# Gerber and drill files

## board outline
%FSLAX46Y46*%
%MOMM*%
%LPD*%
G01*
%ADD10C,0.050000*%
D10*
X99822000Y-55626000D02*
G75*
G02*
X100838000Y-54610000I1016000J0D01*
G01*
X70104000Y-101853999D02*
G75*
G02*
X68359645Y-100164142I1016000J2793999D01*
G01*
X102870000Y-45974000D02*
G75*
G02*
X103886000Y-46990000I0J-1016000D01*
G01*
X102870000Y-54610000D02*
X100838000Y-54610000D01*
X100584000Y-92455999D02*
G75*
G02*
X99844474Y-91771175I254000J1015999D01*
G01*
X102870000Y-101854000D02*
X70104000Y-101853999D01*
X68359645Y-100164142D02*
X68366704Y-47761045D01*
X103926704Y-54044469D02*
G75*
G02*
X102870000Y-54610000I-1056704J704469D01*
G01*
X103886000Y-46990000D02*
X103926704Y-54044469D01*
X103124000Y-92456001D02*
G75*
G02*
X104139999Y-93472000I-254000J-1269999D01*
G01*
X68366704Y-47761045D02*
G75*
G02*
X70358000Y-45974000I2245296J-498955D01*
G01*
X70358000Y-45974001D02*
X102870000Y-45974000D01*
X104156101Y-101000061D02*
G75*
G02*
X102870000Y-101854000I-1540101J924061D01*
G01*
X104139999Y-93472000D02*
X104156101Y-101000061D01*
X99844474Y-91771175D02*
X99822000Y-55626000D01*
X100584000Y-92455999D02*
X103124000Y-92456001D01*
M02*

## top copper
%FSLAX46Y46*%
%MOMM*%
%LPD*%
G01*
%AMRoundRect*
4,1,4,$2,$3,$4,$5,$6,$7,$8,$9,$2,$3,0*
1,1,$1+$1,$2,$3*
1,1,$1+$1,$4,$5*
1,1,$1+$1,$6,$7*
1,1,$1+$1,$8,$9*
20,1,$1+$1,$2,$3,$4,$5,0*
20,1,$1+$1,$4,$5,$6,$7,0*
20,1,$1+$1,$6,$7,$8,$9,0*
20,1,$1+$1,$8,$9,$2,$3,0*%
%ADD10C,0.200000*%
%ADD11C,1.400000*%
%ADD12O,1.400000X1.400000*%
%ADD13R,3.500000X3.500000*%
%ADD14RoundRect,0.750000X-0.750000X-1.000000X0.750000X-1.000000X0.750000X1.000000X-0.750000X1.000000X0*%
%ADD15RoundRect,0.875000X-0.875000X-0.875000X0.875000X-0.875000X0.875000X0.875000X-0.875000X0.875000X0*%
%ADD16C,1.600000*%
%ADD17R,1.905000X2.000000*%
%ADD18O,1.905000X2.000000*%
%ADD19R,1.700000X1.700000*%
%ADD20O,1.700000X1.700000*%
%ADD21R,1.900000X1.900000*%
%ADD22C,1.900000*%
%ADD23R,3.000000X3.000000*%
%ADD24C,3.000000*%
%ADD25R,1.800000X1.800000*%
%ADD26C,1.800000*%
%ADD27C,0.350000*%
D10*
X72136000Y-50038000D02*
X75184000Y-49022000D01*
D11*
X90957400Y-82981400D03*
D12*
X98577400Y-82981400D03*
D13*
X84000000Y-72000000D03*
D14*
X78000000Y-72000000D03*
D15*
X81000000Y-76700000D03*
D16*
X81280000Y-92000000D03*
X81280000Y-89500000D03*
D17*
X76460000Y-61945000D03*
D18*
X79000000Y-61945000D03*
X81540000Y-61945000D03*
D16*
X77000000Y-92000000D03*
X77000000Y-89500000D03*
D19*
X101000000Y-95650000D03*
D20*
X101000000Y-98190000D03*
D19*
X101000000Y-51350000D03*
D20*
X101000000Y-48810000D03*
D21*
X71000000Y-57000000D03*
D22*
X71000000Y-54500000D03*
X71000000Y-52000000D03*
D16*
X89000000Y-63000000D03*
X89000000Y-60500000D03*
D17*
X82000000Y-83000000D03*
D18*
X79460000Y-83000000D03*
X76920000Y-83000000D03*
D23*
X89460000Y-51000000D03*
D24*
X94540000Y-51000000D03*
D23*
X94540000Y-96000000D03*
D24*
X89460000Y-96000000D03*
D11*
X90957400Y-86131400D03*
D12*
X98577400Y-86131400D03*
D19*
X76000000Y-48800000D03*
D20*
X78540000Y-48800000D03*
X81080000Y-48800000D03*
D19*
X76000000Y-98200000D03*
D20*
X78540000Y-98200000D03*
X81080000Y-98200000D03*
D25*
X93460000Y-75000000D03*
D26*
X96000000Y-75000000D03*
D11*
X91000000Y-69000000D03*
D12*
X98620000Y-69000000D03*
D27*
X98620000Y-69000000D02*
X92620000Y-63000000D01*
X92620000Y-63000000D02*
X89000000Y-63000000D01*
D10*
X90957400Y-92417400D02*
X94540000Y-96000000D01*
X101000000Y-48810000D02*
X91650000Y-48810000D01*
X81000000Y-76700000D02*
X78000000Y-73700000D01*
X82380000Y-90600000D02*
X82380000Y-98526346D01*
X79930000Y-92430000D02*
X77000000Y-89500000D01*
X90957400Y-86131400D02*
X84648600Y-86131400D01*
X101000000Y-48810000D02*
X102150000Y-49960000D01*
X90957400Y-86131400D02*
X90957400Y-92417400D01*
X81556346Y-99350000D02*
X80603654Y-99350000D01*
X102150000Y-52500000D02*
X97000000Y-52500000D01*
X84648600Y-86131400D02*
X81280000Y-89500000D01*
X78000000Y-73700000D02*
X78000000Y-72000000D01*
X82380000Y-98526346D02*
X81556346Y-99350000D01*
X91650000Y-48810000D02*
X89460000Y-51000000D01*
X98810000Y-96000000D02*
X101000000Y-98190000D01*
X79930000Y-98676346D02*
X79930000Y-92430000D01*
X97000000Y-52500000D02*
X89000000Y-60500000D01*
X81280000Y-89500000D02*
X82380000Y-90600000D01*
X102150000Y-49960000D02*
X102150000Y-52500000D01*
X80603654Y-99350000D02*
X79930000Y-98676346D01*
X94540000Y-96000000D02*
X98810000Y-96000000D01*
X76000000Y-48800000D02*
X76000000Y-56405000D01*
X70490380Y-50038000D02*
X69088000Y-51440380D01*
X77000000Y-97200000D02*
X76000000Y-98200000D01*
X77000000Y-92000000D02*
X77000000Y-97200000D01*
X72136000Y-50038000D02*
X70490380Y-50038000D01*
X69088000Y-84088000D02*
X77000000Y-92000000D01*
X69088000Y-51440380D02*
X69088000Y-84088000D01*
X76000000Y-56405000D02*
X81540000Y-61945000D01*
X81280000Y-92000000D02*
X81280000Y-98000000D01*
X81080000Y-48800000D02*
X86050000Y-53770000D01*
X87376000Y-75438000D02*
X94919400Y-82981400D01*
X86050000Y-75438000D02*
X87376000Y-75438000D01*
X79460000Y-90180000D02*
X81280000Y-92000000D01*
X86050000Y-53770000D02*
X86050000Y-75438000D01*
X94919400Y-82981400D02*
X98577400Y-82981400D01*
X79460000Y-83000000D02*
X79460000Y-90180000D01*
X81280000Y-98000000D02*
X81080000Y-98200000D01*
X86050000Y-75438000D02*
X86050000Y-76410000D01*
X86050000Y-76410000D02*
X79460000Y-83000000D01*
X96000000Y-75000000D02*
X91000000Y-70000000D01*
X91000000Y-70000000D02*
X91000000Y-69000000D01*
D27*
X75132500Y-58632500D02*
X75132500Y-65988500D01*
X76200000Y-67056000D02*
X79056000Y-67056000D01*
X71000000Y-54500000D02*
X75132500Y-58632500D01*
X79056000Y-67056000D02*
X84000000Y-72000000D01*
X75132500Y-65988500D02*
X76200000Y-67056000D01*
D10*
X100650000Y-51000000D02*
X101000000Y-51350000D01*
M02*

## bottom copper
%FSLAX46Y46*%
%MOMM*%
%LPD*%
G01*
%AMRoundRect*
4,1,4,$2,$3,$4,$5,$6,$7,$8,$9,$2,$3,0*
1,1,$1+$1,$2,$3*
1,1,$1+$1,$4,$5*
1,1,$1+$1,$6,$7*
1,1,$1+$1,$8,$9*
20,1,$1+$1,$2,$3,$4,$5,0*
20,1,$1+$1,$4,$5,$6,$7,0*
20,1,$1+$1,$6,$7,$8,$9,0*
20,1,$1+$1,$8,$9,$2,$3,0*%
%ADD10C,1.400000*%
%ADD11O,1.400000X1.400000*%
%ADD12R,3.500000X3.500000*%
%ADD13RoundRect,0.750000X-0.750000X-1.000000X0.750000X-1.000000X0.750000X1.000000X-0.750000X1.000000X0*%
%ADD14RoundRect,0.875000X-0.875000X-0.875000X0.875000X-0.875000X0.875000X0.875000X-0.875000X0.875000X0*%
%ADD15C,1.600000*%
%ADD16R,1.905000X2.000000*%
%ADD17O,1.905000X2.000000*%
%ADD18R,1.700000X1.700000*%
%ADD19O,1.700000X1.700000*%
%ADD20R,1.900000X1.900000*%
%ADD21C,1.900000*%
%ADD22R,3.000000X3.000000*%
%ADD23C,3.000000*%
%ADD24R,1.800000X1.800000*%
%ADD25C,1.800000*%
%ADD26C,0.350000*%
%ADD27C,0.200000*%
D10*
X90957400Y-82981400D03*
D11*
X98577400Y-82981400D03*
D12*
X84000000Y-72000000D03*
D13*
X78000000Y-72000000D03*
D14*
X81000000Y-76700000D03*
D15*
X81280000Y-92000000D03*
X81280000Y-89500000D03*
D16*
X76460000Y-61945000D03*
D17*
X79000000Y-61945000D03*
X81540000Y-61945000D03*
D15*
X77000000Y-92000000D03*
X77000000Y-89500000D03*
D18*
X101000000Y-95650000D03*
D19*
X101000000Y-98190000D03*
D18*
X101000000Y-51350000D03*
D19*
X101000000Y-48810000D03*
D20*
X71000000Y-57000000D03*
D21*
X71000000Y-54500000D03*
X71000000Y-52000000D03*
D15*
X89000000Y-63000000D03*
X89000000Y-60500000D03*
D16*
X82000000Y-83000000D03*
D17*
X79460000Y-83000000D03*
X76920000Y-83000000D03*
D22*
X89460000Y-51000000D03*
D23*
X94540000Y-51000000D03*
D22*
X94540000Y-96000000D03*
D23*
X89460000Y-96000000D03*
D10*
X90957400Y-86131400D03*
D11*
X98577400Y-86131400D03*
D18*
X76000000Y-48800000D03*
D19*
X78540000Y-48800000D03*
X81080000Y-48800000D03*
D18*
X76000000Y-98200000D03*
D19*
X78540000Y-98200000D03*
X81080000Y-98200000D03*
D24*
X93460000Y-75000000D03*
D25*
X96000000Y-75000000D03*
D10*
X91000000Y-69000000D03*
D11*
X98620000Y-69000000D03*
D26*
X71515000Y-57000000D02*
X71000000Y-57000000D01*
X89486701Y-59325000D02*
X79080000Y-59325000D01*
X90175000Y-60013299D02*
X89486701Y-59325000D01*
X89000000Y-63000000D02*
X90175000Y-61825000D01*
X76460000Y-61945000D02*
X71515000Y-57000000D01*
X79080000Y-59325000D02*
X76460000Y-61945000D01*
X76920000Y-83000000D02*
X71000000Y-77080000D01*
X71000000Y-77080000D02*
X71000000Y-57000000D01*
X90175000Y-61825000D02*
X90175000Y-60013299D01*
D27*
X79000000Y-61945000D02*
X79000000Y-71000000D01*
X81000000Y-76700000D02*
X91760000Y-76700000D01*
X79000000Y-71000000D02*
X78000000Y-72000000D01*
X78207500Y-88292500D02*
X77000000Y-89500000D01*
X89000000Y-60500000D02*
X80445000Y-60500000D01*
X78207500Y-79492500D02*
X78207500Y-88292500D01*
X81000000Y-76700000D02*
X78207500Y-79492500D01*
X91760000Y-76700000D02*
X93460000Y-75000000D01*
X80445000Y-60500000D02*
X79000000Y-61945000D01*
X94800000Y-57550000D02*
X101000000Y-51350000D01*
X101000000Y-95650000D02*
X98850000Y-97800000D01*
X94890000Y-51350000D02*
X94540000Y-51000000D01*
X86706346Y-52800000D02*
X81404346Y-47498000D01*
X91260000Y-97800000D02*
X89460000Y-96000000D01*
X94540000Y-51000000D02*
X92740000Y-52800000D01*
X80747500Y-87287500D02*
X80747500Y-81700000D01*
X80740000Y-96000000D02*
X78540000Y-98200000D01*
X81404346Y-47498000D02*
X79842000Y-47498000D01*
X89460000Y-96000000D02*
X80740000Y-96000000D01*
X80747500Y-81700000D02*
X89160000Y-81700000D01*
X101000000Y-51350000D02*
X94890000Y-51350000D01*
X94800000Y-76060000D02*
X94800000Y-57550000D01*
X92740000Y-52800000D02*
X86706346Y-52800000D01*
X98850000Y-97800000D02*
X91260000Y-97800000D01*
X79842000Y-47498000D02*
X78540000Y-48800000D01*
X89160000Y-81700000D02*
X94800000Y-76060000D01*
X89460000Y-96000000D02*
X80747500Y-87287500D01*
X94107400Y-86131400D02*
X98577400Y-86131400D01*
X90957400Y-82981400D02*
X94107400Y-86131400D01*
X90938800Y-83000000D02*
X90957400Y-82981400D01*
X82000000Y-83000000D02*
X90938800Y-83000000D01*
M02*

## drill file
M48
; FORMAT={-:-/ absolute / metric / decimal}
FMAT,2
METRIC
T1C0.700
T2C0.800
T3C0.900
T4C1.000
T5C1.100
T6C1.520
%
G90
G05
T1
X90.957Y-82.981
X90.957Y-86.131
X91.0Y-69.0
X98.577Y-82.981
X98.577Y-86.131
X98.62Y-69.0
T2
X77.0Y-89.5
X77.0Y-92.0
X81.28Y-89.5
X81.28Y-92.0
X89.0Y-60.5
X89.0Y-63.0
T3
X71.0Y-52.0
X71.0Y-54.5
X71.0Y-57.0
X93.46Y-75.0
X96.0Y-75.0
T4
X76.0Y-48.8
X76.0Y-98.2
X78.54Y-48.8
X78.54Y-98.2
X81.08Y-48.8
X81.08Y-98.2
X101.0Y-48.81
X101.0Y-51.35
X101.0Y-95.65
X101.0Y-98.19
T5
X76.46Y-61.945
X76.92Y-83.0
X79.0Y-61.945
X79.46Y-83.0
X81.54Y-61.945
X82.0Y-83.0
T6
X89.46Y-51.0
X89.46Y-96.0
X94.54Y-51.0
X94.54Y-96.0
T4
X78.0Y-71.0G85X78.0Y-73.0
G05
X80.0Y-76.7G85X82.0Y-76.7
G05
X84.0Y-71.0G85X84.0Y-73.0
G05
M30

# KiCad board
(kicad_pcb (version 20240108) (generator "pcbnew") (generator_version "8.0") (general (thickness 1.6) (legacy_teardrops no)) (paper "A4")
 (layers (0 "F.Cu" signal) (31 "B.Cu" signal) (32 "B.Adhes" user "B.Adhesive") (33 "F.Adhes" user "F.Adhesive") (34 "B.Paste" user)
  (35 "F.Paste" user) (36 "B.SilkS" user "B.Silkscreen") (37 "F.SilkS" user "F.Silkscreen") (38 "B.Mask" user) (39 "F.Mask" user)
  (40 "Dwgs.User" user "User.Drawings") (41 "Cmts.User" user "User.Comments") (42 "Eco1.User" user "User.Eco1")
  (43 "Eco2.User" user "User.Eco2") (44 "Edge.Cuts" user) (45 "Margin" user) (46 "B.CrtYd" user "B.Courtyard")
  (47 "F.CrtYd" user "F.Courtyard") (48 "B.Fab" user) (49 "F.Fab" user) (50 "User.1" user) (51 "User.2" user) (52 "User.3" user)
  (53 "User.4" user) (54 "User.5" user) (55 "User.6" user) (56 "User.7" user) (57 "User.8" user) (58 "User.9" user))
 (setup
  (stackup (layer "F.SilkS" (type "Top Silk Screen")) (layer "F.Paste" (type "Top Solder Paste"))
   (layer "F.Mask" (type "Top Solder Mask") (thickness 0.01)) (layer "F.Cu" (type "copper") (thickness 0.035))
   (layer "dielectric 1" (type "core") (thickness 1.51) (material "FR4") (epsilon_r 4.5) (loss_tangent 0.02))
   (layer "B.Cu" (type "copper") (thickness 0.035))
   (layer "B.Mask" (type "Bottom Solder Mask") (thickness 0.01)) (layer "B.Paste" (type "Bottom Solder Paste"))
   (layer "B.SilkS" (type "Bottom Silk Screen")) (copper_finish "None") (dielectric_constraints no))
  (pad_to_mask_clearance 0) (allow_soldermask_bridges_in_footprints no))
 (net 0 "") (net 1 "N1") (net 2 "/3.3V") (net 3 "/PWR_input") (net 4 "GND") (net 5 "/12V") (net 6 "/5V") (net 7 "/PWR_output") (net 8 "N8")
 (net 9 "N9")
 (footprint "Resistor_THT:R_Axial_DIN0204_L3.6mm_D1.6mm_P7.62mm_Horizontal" (layer "F.Cu") (at 90.9574 82.9814)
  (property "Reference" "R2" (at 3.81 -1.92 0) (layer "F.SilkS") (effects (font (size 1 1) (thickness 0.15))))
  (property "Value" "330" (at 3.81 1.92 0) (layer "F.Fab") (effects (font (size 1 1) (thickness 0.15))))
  (pad "1" thru_hole circle (at 0 0) (size 1.4 1.4) (drill 0.7) (layers "*.Cu" "*.Mask") (remove_unused_layers no) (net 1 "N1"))
  (pad "2" thru_hole oval (at 7.62 0) (size 1.4 1.4) (drill 0.7) (layers "*.Cu" "*.Mask") (remove_unused_layers no) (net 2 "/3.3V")))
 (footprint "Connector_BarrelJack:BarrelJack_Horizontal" (layer "F.Cu") (at 84 72)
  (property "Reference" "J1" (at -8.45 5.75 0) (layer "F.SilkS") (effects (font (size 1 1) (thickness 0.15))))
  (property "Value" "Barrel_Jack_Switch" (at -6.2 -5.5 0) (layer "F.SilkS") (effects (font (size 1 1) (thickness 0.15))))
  (pad "1" thru_hole rect (at 0 0) (size 3.5 3.5) (drill oval 1 3) (layers "*.Cu" "*.Mask") (remove_unused_layers no) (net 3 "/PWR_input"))
  (pad "2" thru_hole roundrect (at -6 0) (size 3 3.5) (drill oval 1 3) (layers "*.Cu" "*.Mask") (remove_unused_layers no)
   (roundrect_rratio 0.25) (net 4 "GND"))
  (pad "3" thru_hole roundrect (at -3 4.7) (size 3.5 3.5) (drill oval 3 1) (layers "*.Cu" "*.Mask") (remove_unused_layers no)
   (roundrect_rratio 0.25) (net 4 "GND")))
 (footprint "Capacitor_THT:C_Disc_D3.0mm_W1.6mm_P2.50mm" (layer "F.Cu") (at 81.28 92 90)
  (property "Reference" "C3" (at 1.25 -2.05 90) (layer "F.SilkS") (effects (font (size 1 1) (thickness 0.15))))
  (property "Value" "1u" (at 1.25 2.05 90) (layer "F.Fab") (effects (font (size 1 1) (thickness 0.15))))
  (pad "1" thru_hole circle (at 0 0 90) (size 1.6 1.6) (drill 0.8) (layers "*.Cu" "*.Mask") (remove_unused_layers no) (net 2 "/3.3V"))
  (pad "2" thru_hole circle (at 2.5 0 90) (size 1.6 1.6) (drill 0.8) (layers "*.Cu" "*.Mask") (remove_unused_layers no) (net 4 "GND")))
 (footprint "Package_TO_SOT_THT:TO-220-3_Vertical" (layer "F.Cu") (at 76.46 61.945)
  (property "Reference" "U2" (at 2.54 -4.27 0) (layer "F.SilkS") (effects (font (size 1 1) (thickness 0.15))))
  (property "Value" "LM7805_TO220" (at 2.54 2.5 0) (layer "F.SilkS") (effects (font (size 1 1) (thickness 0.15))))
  (pad "1" thru_hole rect (at 0 0) (size 1.905 2) (drill 1.1) (layers "*.Cu" "*.Mask") (remove_unused_layers no) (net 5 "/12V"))
  (pad "2" thru_hole oval (at 2.54 0) (size 1.905 2) (drill 1.1) (layers "*.Cu" "*.Mask") (remove_unused_layers no) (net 4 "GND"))
  (pad "3" thru_hole oval (at 5.08 0) (size 1.905 2) (drill 1.1) (layers "*.Cu" "*.Mask") (remove_unused_layers no) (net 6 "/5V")))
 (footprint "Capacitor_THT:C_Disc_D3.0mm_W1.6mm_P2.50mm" (layer "F.Cu") (at 77 92 90)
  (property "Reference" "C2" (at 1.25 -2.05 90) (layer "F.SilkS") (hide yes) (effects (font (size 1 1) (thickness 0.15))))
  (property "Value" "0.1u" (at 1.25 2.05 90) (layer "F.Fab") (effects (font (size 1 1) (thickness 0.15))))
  (pad "1" thru_hole circle (at 0 0 90) (size 1.6 1.6) (drill 0.8) (layers "*.Cu" "*.Mask") (remove_unused_layers no) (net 6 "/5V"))
  (pad "2" thru_hole circle (at 2.5 0 90) (size 1.6 1.6) (drill 0.8) (layers "*.Cu" "*.Mask") (remove_unused_layers no) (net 4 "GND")))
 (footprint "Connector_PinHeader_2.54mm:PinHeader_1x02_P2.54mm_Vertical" (layer "F.Cu") (at 101 95.65)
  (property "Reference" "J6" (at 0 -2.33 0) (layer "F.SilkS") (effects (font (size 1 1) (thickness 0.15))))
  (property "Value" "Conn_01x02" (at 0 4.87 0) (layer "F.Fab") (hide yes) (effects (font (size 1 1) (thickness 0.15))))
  (pad "1" thru_hole rect (at 0 0) (size 1.7 1.7) (drill 1) (layers "*.Cu" "*.Mask") (remove_unused_layers no) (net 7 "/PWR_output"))
  (pad "2" thru_hole oval (at 0 2.54) (size 1.7 1.7) (drill 1) (layers "*.Cu" "*.Mask") (remove_unused_layers no) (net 4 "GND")))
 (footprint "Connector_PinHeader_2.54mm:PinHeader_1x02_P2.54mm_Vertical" (layer "F.Cu") (at 101 51.35 180)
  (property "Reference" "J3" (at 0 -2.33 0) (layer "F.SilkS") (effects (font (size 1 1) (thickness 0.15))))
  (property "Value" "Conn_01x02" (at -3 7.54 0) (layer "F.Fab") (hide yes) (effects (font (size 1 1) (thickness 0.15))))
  (pad "1" thru_hole rect (at 0 0 180) (size 1.7 1.7) (drill 1) (layers "*.Cu" "*.Mask") (remove_unused_layers no) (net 7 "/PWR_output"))
  (pad "2" thru_hole oval (at 0 2.54 180) (size 1.7 1.7) (drill 1) (layers "*.Cu" "*.Mask") (remove_unused_layers no) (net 4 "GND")))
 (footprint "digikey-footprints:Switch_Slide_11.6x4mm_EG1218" (layer "F.Cu") (at 71 57 90)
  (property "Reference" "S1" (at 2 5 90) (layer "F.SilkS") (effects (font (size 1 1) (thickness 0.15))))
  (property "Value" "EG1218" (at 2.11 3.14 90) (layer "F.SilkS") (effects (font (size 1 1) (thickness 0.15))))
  (pad "1" thru_hole rect (at 0 0 90) (size 1.9 1.9) (drill 0.9) (layers "*.Cu" "*.Mask") (remove_unused_layers no) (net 5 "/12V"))
  (pad "2" thru_hole circle (at 2.5 0 90) (size 1.9 1.9) (drill 0.9) (layers "*.Cu" "*.Mask") (remove_unused_layers no) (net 3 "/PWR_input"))
  (pad "3" thru_hole circle (at 5 0 90) (size 1.9 1.9) (drill 0.9) (layers "*.Cu" "*.Mask") (remove_unused_layers no) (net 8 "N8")))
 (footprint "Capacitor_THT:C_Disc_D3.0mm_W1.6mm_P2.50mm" (layer "F.Cu") (at 89 63 90)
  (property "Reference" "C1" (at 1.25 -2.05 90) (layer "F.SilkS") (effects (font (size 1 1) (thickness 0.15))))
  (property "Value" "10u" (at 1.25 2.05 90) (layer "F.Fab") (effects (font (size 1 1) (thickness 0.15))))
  (pad "1" thru_hole circle (at 0 0 90) (size 1.6 1.6) (drill 0.8) (layers "*.Cu" "*.Mask") (remove_unused_layers no) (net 5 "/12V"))
  (pad "2" thru_hole circle (at 2.5 0 90) (size 1.6 1.6) (drill 0.8) (layers "*.Cu" "*.Mask") (remove_unused_layers no) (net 4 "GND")))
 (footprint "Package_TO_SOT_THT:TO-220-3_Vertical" (layer "F.Cu") (at 82 83 180)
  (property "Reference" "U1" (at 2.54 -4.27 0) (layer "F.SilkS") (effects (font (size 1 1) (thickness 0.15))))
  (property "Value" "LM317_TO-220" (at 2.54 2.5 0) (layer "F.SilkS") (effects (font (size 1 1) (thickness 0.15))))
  (pad "1" thru_hole rect (at 0 0 180) (size 1.905 2) (drill 1.1) (layers "*.Cu" "*.Mask") (remove_unused_layers no) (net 1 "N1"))
  (pad "2" thru_hole oval (at 2.54 0 180) (size 1.905 2) (drill 1.1) (layers "*.Cu" "*.Mask") (remove_unused_layers no) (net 2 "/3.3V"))
  (pad "3" thru_hole oval (at 5.08 0 180) (size 1.905 2) (drill 1.1) (layers "*.Cu" "*.Mask") (remove_unused_layers no) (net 5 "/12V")))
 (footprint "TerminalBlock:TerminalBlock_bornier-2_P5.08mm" (layer "F.Cu") (at 89.46 51)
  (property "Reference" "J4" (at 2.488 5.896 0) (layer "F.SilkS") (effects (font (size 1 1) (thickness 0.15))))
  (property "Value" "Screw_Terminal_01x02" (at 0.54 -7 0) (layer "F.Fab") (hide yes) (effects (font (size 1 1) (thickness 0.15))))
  (pad "1" thru_hole rect (at 0 0) (size 3 3) (drill 1.52) (layers "*.Cu" "*.Mask") (remove_unused_layers no) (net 4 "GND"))
  (pad "2" thru_hole circle (at 5.08 0) (size 3 3) (drill 1.52) (layers "*.Cu" "*.Mask") (remove_unused_layers no) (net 7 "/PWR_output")))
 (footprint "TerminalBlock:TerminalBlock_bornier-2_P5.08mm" (layer "F.Cu") (at 94.54 96 180)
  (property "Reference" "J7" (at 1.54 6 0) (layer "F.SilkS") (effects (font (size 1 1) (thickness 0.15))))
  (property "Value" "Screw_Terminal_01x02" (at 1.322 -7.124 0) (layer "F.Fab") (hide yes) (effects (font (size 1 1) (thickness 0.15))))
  (pad "1" thru_hole rect (at 0 0 180) (size 3 3) (drill 1.52) (layers "*.Cu" "*.Mask") (remove_unused_layers no) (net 4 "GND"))
  (pad "2" thru_hole circle (at 5.08 0 180) (size 3 3) (drill 1.52) (layers "*.Cu" "*.Mask") (remove_unused_layers no) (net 7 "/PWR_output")))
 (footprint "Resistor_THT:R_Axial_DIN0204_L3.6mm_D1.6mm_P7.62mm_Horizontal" (layer "F.Cu") (at 90.9574 86.1314)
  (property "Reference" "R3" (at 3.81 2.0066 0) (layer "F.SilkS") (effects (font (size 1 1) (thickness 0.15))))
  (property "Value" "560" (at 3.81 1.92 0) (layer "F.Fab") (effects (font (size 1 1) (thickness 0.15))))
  (pad "1" thru_hole circle (at 0 0) (size 1.4 1.4) (drill 0.7) (layers "*.Cu" "*.Mask") (remove_unused_layers no) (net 4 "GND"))
  (pad "2" thru_hole oval (at 7.62 0) (size 1.4 1.4) (drill 0.7) (layers "*.Cu" "*.Mask") (remove_unused_layers no) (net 1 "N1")))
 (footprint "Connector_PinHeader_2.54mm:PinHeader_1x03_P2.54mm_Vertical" (layer "F.Cu") (at 76 48.8 90)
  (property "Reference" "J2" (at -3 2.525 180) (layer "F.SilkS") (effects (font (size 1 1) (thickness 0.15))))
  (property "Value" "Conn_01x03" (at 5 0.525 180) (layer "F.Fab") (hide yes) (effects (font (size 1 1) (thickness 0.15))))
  (pad "1" thru_hole rect (at 0 0 90) (size 1.7 1.7) (drill 1) (layers "*.Cu" "*.Mask") (remove_unused_layers no) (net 6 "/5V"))
  (pad "2" thru_hole oval (at 0 2.54 90) (size 1.7 1.7) (drill 1) (layers "*.Cu" "*.Mask") (remove_unused_layers no) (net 7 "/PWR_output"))
  (pad "3" thru_hole oval (at 0 5.08 90) (size 1.7 1.7) (drill 1) (layers "*.Cu" "*.Mask") (remove_unused_layers no) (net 2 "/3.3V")))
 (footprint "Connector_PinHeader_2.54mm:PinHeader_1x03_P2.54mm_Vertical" (layer "F.Cu") (at 76 98.2 90)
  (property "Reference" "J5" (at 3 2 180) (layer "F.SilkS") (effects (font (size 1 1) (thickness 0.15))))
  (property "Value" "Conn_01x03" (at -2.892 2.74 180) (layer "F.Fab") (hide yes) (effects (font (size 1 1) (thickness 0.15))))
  (pad "1" thru_hole rect (at 0 0 90) (size 1.7 1.7) (drill 1) (layers "*.Cu" "*.Mask") (remove_unused_layers no) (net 6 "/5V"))
  (pad "2" thru_hole oval (at 0 2.54 90) (size 1.7 1.7) (drill 1) (layers "*.Cu" "*.Mask") (remove_unused_layers no) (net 7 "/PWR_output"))
  (pad "3" thru_hole oval (at 0 5.08 90) (size 1.7 1.7) (drill 1) (layers "*.Cu" "*.Mask") (remove_unused_layers no) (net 2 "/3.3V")))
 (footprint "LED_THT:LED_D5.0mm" (layer "F.Cu") (at 93.46 75)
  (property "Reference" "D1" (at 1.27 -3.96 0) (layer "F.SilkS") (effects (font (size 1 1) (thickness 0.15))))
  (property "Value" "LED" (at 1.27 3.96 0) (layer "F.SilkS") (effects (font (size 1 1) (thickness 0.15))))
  (pad "1" thru_hole rect (at 0 0) (size 1.8 1.8) (drill 0.9) (layers "*.Cu" "*.Mask") (remove_unused_layers no) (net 4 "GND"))
  (pad "2" thru_hole circle (at 2.54 0) (size 1.8 1.8) (drill 0.9) (layers "*.Cu" "*.Mask") (remove_unused_layers no) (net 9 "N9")))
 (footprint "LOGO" (layer "F.Cu") (at 96.52 60.96 90)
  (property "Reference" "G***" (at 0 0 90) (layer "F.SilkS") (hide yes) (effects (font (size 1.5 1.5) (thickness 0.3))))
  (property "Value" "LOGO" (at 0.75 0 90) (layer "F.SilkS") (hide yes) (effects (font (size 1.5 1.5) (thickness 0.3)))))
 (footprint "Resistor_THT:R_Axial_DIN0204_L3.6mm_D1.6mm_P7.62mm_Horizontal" (layer "F.Cu") (at 91 69)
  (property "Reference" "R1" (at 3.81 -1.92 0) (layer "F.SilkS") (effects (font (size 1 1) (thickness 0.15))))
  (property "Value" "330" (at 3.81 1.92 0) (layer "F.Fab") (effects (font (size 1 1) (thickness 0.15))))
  (pad "1" thru_hole circle (at 0 0) (size 1.4 1.4) (drill 0.7) (layers "*.Cu" "*.Mask") (remove_unused_layers no) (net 9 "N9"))
  (pad "2" thru_hole oval (at 7.62 0) (size 1.4 1.4) (drill 0.7) (layers "*.Cu" "*.Mask") (remove_unused_layers no) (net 5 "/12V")))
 (gr_line (start 72.136 50.038) (end 75.184 49.022) (stroke (width 0.2) (type default)) (layer "F.Cu") (net 6))
 (gr_arc (start 99.822 55.626) (mid 100.11958 54.90758) (end 100.838 54.61) (stroke (width 0.05) (type default)) (layer "Edge.Cuts"))
 (gr_arc (start 70.104 101.853999) (mid 69.051397 101.195315) (end 68.359645 100.164142) (stroke (width 0.05) (type default))
  (layer "Edge.Cuts"))
 (gr_arc (start 102.87 45.974) (mid 103.58842 46.27158) (end 103.886 46.99) (stroke (width 0.05) (type default)) (layer "Edge.Cuts"))
 (gr_line (start 102.87 54.61) (end 100.838 54.61) (stroke (width 0.05) (type default)) (layer "Edge.Cuts"))
 (gr_arc (start 100.584 92.455999) (mid 100.126434 92.208403) (end 99.844474 91.771175) (stroke (width 0.05) (type default))
  (layer "Edge.Cuts"))
 (gr_line (start 102.87 101.854) (end 70.104 101.853999) (stroke (width 0.05) (type default)) (layer "Edge.Cuts"))
 (gr_line (start 68.359645 100.164142) (end 68.366704 47.761045) (stroke (width 0.05) (type default)) (layer "Edge.Cuts"))
 (gr_arc (start 103.926704 54.044469) (mid 103.46926 54.459727) (end 102.87 54.61) (stroke (width 0.05) (type default)) (layer "Edge.Cuts"))
 (gr_line (start 103.886 46.99) (end 103.926704 54.044469) (stroke (width 0.05) (type default)) (layer "Edge.Cuts"))
 (gr_arc (start 103.124 92.456001) (mid 103.785809 92.810191) (end 104.139999 93.472) (stroke (width 0.05) (type default))
  (layer "Edge.Cuts"))
 (gr_arc (start 68.366704 47.761045) (mid 69.07577 46.548186) (end 70.358 45.974001) (stroke (width 0.05) (type default))
  (layer "Edge.Cuts"))
 (gr_line (start 70.358 45.974001) (end 102.87 45.974) (stroke (width 0.05) (type default)) (layer "Edge.Cuts"))
 (gr_arc (start 104.156101 101.000061) (mid 103.60948 101.572261) (end 102.87 101.854) (stroke (width 0.05) (type default))
  (layer "Edge.Cuts"))
 (gr_line (start 104.139999 93.472) (end 104.156101 101.000061) (stroke (width 0.05) (type default)) (layer "Edge.Cuts"))
 (gr_line (start 99.844474 91.771175) (end 99.822 55.626) (stroke (width 0.05) (type default)) (layer "Edge.Cuts"))
 (gr_line (start 100.584 92.455999) (end 103.124 92.456001) (stroke (width 0.05) (type default)) (layer "Edge.Cuts"))
 (segment (start 98.62 69) (end 92.62 63) (width 0.35) (layer "F.Cu") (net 5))
 (segment (start 92.62 63) (end 89 63) (width 0.35) (layer "F.Cu") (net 5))
 (segment (start 71.515 57) (end 71 57) (width 0.35) (layer "B.Cu") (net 5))
 (segment (start 89.486701 59.325) (end 79.08 59.325) (width 0.35) (layer "B.Cu") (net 5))
 (segment (start 90.175 60.013299) (end 89.486701 59.325) (width 0.35) (layer "B.Cu") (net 5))
 (segment (start 89 63) (end 90.175 61.825) (width 0.35) (layer "B.Cu") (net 5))
 (segment (start 76.46 61.945) (end 71.515 57) (width 0.35) (layer "B.Cu") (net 5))
 (segment (start 79.08 59.325) (end 76.46 61.945) (width 0.35) (layer "B.Cu") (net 5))
 (segment (start 76.92 83) (end 71 77.08) (width 0.35) (layer "B.Cu") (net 5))
 (segment (start 71 77.08) (end 71 57) (width 0.35) (layer "B.Cu") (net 5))
 (segment (start 90.175 61.825) (end 90.175 60.013299) (width 0.35) (layer "B.Cu") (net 5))
 (segment (start 90.9574 92.4174) (end 94.54 96) (width 0.2) (layer "F.Cu") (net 4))
 (segment (start 101 48.81) (end 91.65 48.81) (width 0.2) (layer "F.Cu") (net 4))
 (segment (start 81 76.7) (end 78 73.7) (width 0.2) (layer "F.Cu") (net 4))
 (segment (start 82.38 90.6) (end 82.38 98.526346) (width 0.2) (layer "F.Cu") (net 4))
 (segment (start 79.93 92.43) (end 77 89.5) (width 0.2) (layer "F.Cu") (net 4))
 (segment (start 90.9574 86.1314) (end 84.6486 86.1314) (width 0.2) (layer "F.Cu") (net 4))
 (segment (start 101 48.81) (end 102.15 49.96) (width 0.2) (layer "F.Cu") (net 4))
 (segment (start 90.9574 86.1314) (end 90.9574 92.4174) (width 0.2) (layer "F.Cu") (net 4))
 (segment (start 81.556346 99.35) (end 80.603654 99.35) (width 0.2) (layer "F.Cu") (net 4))
 (segment (start 102.15 52.5) (end 97 52.5) (width 0.2) (layer "F.Cu") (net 4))
 (segment (start 84.6486 86.1314) (end 81.28 89.5) (width 0.2) (layer "F.Cu") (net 4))
 (segment (start 78 73.7) (end 78 72) (width 0.2) (layer "F.Cu") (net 4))
 (segment (start 82.38 98.526346) (end 81.556346 99.35) (width 0.2) (layer "F.Cu") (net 4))
 (segment (start 91.65 48.81) (end 89.46 51) (width 0.2) (layer "F.Cu") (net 4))
 (segment (start 98.81 96) (end 101 98.19) (width 0.2) (layer "F.Cu") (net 4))
 (segment (start 79.93 98.676346) (end 79.93 92.43) (width 0.2) (layer "F.Cu") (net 4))
 (segment (start 97 52.5) (end 89 60.5) (width 0.2) (layer "F.Cu") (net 4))
 (segment (start 81.28 89.5) (end 82.38 90.6) (width 0.2) (layer "F.Cu") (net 4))
 (segment (start 102.15 49.96) (end 102.15 52.5) (width 0.2) (layer "F.Cu") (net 4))
 (segment (start 80.603654 99.35) (end 79.93 98.676346) (width 0.2) (layer "F.Cu") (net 4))
 (segment (start 94.54 96) (end 98.81 96) (width 0.2) (layer "F.Cu") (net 4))
 (segment (start 79 61.945) (end 79 71) (width 0.2) (layer "B.Cu") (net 4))
 (segment (start 81 76.7) (end 91.76 76.7) (width 0.2) (layer "B.Cu") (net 4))
 (segment (start 79 71) (end 78 72) (width 0.2) (layer "B.Cu") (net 4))
 (segment (start 78.2075 88.2925) (end 77 89.5) (width 0.2) (layer "B.Cu") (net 4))
 (segment (start 89 60.5) (end 80.445 60.5) (width 0.2) (layer "B.Cu") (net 4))
 (segment (start 78.2075 79.4925) (end 78.2075 88.2925) (width 0.2) (layer "B.Cu") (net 4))
 (segment (start 81 76.7) (end 78.2075 79.4925) (width 0.2) (layer "B.Cu") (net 4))
 (segment (start 91.76 76.7) (end 93.46 75) (width 0.2) (layer "B.Cu") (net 4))
 (segment (start 80.445 60.5) (end 79 61.945) (width 0.2) (layer "B.Cu") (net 4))
 (segment (start 76 48.8) (end 76 56.405) (width 0.2) (layer "F.Cu") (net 6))
 (segment (start 70.49038 50.038) (end 69.088 51.44038) (width 0.2) (layer "F.Cu") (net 6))
 (segment (start 77 97.2) (end 76 98.2) (width 0.2) (layer "F.Cu") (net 6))
 (segment (start 77 92) (end 77 97.2) (width 0.2) (layer "F.Cu") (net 6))
 (segment (start 72.136 50.038) (end 70.49038 50.038) (width 0.2) (layer "F.Cu") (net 6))
 (segment (start 69.088 84.088) (end 77 92) (width 0.2) (layer "F.Cu") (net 6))
 (segment (start 69.088 51.44038) (end 69.088 84.088) (width 0.2) (layer "F.Cu") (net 6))
 (segment (start 76 56.405) (end 81.54 61.945) (width 0.2) (layer "F.Cu") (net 6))
 (segment (start 81.28 92) (end 81.28 98) (width 0.2) (layer "F.Cu") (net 2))
 (segment (start 81.08 48.8) (end 86.05 53.77) (width 0.2) (layer "F.Cu") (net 2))
 (segment (start 87.376 75.438) (end 94.9194 82.9814) (width 0.2) (layer "F.Cu") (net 2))
 (segment (start 86.05 75.438) (end 87.376 75.438) (width 0.2) (layer "F.Cu") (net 2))
 (segment (start 79.46 90.18) (end 81.28 92) (width 0.2) (layer "F.Cu") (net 2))
 (segment (start 86.05 53.77) (end 86.05 75.438) (width 0.2) (layer "F.Cu") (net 2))
 (segment (start 94.9194 82.9814) (end 98.5774 82.9814) (width 0.2) (layer "F.Cu") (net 2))
 (segment (start 79.46 83) (end 79.46 90.18) (width 0.2) (layer "F.Cu") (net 2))
 (segment (start 81.28 98) (end 81.08 98.2) (width 0.2) (layer "F.Cu") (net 2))
 (segment (start 86.05 75.438) (end 86.05 76.41) (width 0.2) (layer "F.Cu") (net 2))
 (segment (start 86.05 76.41) (end 79.46 83) (width 0.2) (layer "F.Cu") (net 2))
 (segment (start 96 75) (end 91 70) (width 0.2) (layer "F.Cu") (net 9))
 (segment (start 91 70) (end 91 69) (width 0.2) (layer "F.Cu") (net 9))
 (segment (start 75.1325 58.6325) (end 75.1325 65.9885) (width 0.35) (layer "F.Cu") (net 3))
 (segment (start 76.2 67.056) (end 79.056 67.056) (width 0.35) (layer "F.Cu") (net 3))
 (segment (start 71 54.5) (end 75.1325 58.6325) (width 0.35) (layer "F.Cu") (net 3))
 (segment (start 79.056 67.056) (end 84 72) (width 0.35) (layer "F.Cu") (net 3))
 (segment (start 75.1325 65.9885) (end 76.2 67.056) (width 0.35) (layer "F.Cu") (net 3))
 (segment (start 100.65 51) (end 101 51.35) (width 0.2) (layer "F.Cu") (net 7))
 (segment (start 94.8 57.55) (end 101 51.35) (width 0.2) (layer "B.Cu") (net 7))
 (segment (start 101 95.65) (end 98.85 97.8) (width 0.2) (layer "B.Cu") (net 7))
 (segment (start 94.89 51.35) (end 94.54 51) (width 0.2) (layer "B.Cu") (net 7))
 (segment (start 86.706346 52.8) (end 81.404346 47.498) (width 0.2) (layer "B.Cu") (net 7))
 (segment (start 91.26 97.8) (end 89.46 96) (width 0.2) (layer "B.Cu") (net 7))
 (segment (start 94.54 51) (end 92.74 52.8) (width 0.2) (layer "B.Cu") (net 7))
 (segment (start 80.7475 87.2875) (end 80.7475 81.7) (width 0.2) (layer "B.Cu") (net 7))
 (segment (start 80.74 96) (end 78.54 98.2) (width 0.2) (layer "B.Cu") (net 7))
 (segment (start 81.404346 47.498) (end 79.842 47.498) (width 0.2) (layer "B.Cu") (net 7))
 (segment (start 89.46 96) (end 80.74 96) (width 0.2) (layer "B.Cu") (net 7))
 (segment (start 80.7475 81.7) (end 89.16 81.7) (width 0.2) (layer "B.Cu") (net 7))
 (segment (start 101 51.35) (end 94.89 51.35) (width 0.2) (layer "B.Cu") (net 7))
 (segment (start 94.8 76.06) (end 94.8 57.55) (width 0.2) (layer "B.Cu") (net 7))
 (segment (start 92.74 52.8) (end 86.706346 52.8) (width 0.2) (layer "B.Cu") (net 7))
 (segment (start 98.85 97.8) (end 91.26 97.8) (width 0.2) (layer "B.Cu") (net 7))
 (segment (start 79.842 47.498) (end 78.54 48.8) (width 0.2) (layer "B.Cu") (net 7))
 (segment (start 89.16 81.7) (end 94.8 76.06) (width 0.2) (layer "B.Cu") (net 7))
 (segment (start 89.46 96) (end 80.7475 87.2875) (width 0.2) (layer "B.Cu") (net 7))
 (segment (start 94.1074 86.1314) (end 98.5774 86.1314) (width 0.2) (layer "B.Cu") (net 1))
 (segment (start 90.9574 82.9814) (end 94.1074 86.1314) (width 0.2) (layer "B.Cu") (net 1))
 (segment (start 90.9388 83) (end 90.9574 82.9814) (width 0.2) (layer "B.Cu") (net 1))
 (segment (start 82 83) (end 90.9388 83) (width 0.2) (layer "B.Cu") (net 1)))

